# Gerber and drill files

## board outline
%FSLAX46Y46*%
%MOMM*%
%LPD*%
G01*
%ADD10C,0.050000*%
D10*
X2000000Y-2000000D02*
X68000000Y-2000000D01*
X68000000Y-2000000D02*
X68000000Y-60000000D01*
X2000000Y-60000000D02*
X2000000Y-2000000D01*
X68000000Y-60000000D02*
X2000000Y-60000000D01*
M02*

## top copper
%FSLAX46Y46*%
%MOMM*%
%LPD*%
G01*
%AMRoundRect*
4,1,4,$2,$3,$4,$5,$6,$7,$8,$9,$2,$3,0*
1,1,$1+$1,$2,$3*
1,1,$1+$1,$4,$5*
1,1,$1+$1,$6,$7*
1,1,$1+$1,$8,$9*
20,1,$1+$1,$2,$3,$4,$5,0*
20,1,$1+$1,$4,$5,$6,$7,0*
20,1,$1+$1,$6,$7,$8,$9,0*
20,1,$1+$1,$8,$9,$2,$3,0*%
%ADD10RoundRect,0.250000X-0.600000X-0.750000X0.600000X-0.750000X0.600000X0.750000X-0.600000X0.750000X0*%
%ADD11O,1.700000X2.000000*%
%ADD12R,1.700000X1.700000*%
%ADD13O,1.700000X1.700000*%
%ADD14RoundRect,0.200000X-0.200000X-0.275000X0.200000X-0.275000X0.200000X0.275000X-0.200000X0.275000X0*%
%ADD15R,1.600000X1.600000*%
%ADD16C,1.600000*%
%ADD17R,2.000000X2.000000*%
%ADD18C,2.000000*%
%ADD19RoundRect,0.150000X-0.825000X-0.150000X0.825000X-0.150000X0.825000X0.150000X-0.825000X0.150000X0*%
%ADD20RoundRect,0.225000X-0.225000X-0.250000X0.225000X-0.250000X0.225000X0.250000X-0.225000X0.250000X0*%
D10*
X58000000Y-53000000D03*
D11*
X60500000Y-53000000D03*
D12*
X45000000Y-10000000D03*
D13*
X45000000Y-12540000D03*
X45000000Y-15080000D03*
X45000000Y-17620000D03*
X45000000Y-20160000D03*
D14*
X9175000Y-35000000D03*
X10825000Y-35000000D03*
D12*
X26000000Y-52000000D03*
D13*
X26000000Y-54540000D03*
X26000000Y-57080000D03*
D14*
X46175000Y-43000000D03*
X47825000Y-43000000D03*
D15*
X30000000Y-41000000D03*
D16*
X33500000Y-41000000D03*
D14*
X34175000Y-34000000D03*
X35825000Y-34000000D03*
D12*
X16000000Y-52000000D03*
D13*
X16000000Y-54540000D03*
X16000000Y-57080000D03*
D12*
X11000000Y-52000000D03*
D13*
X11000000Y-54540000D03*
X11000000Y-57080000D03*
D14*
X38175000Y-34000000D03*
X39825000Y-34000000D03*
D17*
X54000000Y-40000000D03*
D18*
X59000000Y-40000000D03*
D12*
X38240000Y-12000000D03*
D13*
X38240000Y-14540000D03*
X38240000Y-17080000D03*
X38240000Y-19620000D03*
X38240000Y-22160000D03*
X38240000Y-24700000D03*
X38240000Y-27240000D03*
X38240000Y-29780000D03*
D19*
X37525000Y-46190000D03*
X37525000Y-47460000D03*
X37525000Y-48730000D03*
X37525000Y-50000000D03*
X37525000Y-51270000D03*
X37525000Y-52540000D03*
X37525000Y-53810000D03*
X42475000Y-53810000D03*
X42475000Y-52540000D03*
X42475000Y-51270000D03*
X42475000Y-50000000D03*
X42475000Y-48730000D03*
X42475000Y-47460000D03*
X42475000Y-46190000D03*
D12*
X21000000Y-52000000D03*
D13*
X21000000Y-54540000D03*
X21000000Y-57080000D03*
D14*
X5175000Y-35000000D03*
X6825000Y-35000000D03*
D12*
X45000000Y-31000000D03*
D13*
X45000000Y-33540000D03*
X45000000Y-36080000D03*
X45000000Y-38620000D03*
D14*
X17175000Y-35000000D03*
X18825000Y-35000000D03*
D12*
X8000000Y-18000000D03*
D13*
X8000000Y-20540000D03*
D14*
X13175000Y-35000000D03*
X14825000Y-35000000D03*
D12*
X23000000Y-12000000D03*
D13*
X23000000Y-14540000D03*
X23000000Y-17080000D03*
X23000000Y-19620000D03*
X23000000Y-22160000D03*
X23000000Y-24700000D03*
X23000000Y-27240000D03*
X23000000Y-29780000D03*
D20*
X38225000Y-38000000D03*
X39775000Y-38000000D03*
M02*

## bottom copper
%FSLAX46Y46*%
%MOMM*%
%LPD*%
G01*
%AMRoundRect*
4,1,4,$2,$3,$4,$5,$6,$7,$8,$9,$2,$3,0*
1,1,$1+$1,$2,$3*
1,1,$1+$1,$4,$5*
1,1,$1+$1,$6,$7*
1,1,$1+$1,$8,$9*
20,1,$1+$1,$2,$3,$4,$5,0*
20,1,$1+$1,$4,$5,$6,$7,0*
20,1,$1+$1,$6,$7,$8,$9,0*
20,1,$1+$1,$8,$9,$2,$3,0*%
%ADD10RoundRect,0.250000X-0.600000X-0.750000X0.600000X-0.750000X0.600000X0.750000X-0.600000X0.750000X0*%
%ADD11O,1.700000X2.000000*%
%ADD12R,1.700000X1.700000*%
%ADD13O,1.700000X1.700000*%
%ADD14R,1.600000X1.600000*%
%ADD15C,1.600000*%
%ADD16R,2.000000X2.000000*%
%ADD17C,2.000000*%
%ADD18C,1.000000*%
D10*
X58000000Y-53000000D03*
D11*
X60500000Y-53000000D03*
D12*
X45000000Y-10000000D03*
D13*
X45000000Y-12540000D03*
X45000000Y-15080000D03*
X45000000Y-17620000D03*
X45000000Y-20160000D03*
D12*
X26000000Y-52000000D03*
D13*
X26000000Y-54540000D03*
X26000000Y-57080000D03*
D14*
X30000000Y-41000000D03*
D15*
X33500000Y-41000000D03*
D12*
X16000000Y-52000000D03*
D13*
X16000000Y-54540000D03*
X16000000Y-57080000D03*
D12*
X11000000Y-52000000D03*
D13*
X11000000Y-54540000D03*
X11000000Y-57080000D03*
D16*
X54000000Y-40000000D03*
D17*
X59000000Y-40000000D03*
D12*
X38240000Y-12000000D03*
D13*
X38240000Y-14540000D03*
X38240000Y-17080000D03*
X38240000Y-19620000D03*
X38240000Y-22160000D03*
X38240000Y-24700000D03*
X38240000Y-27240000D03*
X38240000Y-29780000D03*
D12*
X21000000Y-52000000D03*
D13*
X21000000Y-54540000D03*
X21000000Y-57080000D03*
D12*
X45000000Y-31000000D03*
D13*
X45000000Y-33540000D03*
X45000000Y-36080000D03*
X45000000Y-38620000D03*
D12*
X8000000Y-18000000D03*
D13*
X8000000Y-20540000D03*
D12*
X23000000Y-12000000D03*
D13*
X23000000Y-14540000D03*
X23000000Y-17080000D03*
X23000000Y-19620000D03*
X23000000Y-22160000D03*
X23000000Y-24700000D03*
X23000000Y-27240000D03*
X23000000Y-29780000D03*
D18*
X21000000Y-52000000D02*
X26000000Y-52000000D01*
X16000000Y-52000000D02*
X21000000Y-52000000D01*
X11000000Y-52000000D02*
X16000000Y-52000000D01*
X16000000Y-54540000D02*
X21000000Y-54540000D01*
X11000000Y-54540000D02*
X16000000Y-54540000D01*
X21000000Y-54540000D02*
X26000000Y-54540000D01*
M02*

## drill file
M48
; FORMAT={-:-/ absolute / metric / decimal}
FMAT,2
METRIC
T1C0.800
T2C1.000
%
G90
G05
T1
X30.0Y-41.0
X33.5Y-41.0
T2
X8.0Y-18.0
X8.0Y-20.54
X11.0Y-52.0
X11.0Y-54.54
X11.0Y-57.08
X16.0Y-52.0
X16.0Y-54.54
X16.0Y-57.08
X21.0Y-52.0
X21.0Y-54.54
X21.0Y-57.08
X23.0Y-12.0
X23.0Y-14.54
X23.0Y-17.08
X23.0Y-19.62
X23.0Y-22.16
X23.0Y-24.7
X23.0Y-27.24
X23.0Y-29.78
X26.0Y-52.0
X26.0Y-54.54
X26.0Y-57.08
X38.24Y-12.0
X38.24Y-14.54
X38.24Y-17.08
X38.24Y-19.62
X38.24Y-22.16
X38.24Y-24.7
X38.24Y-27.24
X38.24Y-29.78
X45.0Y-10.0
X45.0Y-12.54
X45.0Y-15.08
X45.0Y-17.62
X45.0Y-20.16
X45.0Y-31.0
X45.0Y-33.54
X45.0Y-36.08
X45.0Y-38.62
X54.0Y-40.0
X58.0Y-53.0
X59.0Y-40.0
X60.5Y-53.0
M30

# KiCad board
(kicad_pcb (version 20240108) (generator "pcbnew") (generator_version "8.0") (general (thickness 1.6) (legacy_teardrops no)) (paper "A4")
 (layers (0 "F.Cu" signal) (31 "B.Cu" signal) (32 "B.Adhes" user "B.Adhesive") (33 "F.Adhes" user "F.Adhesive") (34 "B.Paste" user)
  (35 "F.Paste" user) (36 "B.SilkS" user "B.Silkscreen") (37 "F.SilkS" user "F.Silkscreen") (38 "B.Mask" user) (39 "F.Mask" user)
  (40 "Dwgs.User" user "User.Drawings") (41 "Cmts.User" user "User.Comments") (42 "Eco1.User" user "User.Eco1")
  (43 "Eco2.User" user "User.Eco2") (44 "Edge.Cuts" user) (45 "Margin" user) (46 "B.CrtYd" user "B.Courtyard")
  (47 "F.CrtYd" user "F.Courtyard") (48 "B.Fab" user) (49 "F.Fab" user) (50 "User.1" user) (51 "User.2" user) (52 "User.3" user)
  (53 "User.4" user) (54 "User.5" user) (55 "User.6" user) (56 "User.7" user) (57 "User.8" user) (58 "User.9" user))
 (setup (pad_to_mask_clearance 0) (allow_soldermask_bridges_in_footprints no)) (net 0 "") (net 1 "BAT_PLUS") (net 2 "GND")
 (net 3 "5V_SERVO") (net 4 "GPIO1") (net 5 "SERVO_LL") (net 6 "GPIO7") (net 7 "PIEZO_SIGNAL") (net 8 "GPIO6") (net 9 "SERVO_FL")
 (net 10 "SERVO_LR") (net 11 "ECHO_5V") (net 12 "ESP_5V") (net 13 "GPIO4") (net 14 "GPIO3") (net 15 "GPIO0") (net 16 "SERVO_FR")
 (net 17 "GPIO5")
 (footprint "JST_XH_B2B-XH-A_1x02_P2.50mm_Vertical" (layer "F.Cu") (at 58 53)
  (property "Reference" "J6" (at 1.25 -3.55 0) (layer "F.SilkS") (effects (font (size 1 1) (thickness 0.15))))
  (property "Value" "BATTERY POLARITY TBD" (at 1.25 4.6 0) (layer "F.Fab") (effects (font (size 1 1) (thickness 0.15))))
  (pad "1" thru_hole roundrect (at 0 0) (size 1.7 2) (drill 1) (layers "*.Cu" "*.Mask") (remove_unused_layers no)
   (roundrect_rratio 0.147059) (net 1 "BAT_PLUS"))
  (pad "2" thru_hole oval (at 2.5 0) (size 1.7 2) (drill 1) (layers "*.Cu" "*.Mask") (remove_unused_layers no) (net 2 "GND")))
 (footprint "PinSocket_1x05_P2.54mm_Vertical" (layer "F.Cu") (at 45 10)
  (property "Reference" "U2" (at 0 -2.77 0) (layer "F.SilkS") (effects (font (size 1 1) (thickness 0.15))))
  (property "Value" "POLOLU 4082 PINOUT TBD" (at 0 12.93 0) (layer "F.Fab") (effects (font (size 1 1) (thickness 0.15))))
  (pad "1" thru_hole rect (at 0 0) (size 1.7 1.7) (drill 1) (layers "*.Cu" "*.Mask") (remove_unused_layers no))
  (pad "2" thru_hole oval (at 0 2.54) (size 1.7 1.7) (drill 1) (layers "*.Cu" "*.Mask") (remove_unused_layers no) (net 1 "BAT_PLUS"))
  (pad "3" thru_hole oval (at 0 5.08) (size 1.7 1.7) (drill 1) (layers "*.Cu" "*.Mask") (remove_unused_layers no) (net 2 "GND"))
  (pad "4" thru_hole oval (at 0 7.62) (size 1.7 1.7) (drill 1) (layers "*.Cu" "*.Mask") (remove_unused_layers no) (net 2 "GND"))
  (pad "5" thru_hole oval (at 0 10.16) (size 1.7 1.7) (drill 1) (layers "*.Cu" "*.Mask") (remove_unused_layers no) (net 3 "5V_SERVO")))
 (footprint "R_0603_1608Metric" (layer "F.Cu") (at 10 35)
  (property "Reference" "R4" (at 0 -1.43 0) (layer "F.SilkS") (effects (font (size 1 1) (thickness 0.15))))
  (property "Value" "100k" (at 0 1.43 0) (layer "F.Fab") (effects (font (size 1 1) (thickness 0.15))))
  (pad "1" smd roundrect (at -0.825 0) (size 0.8 0.95) (layers "F.Cu" "F.Paste" "F.Mask") (roundrect_rratio 0.25) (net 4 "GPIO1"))
  (pad "2" smd roundrect (at 0.825 0) (size 0.8 0.95) (layers "F.Cu" "F.Paste" "F.Mask") (roundrect_rratio 0.25) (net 2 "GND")))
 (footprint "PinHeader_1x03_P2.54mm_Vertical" (layer "F.Cu") (at 26 52)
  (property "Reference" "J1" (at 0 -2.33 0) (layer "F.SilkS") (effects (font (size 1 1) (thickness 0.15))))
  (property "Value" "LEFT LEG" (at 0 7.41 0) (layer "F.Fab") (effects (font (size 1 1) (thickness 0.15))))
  (pad "1" thru_hole rect (at 0 0) (size 1.7 1.7) (drill 1) (layers "*.Cu" "*.Mask") (remove_unused_layers no) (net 2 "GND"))
  (pad "2" thru_hole oval (at 0 2.54) (size 1.7 1.7) (drill 1) (layers "*.Cu" "*.Mask") (remove_unused_layers no) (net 3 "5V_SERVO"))
  (pad "3" thru_hole oval (at 0 5.08) (size 1.7 1.7) (drill 1) (layers "*.Cu" "*.Mask") (remove_unused_layers no) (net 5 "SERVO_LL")))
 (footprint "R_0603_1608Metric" (layer "F.Cu") (at 47 43)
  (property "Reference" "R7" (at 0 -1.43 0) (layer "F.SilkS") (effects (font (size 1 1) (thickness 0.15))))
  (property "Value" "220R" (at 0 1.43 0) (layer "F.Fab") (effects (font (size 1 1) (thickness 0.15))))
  (pad "1" smd roundrect (at -0.825 0) (size 0.8 0.95) (layers "F.Cu" "F.Paste" "F.Mask") (roundrect_rratio 0.25) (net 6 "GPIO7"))
  (pad "2" smd roundrect (at 0.825 0) (size 0.8 0.95) (layers "F.Cu" "F.Paste" "F.Mask") (roundrect_rratio 0.25) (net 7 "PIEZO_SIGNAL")))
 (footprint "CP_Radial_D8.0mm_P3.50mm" (layer "F.Cu") (at 30 41)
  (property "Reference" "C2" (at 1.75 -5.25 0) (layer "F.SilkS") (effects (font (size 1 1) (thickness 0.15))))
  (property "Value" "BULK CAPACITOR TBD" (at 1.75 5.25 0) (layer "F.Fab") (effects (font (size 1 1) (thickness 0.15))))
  (pad "1" thru_hole rect (at 0 0) (size 1.6 1.6) (drill 0.8) (layers "*.Cu" "*.Mask") (remove_unused_layers no) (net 3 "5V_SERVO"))
  (pad "2" thru_hole circle (at 3.5 0) (size 1.6 1.6) (drill 0.8) (layers "*.Cu" "*.Mask") (remove_unused_layers no) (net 2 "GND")))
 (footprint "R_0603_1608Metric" (layer "F.Cu") (at 35 34)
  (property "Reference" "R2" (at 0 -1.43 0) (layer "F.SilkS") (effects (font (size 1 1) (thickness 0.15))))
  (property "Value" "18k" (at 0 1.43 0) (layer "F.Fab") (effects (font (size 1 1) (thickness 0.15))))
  (pad "1" smd roundrect (at -0.825 0) (size 0.8 0.95) (layers "F.Cu" "F.Paste" "F.Mask") (roundrect_rratio 0.25) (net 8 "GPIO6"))
  (pad "2" smd roundrect (at 0.825 0) (size 0.8 0.95) (layers "F.Cu" "F.Paste" "F.Mask") (roundrect_rratio 0.25) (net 2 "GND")))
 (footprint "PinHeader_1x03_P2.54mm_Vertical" (layer "F.Cu") (at 16 52)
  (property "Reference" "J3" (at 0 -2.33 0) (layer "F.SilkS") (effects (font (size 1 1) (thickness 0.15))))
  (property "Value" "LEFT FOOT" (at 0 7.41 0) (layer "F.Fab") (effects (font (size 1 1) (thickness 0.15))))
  (pad "1" thru_hole rect (at 0 0) (size 1.7 1.7) (drill 1) (layers "*.Cu" "*.Mask") (remove_unused_layers no) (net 2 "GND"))
  (pad "2" thru_hole oval (at 0 2.54) (size 1.7 1.7) (drill 1) (layers "*.Cu" "*.Mask") (remove_unused_layers no) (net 3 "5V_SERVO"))
  (pad "3" thru_hole oval (at 0 5.08) (size 1.7 1.7) (drill 1) (layers "*.Cu" "*.Mask") (remove_unused_layers no) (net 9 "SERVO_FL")))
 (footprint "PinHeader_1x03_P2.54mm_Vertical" (layer "F.Cu") (at 11 52)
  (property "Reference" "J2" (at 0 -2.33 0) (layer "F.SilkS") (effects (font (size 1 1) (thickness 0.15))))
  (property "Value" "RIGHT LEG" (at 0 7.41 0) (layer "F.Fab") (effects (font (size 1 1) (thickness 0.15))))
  (pad "1" thru_hole rect (at 0 0) (size 1.7 1.7) (drill 1) (layers "*.Cu" "*.Mask") (remove_unused_layers no) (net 2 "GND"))
  (pad "2" thru_hole oval (at 0 2.54) (size 1.7 1.7) (drill 1) (layers "*.Cu" "*.Mask") (remove_unused_layers no) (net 3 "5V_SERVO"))
  (pad "3" thru_hole oval (at 0 5.08) (size 1.7 1.7) (drill 1) (layers "*.Cu" "*.Mask") (remove_unused_layers no) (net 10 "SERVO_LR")))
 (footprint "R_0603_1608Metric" (layer "F.Cu") (at 39 34)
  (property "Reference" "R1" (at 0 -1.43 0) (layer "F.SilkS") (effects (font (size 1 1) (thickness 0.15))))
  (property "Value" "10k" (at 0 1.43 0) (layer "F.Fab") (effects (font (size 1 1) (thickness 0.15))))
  (pad "1" smd roundrect (at -0.825 0) (size 0.8 0.95) (layers "F.Cu" "F.Paste" "F.Mask") (roundrect_rratio 0.25) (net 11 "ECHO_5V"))
  (pad "2" smd roundrect (at 0.825 0) (size 0.8 0.95) (layers "F.Cu" "F.Paste" "F.Mask") (roundrect_rratio 0.25) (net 8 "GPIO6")))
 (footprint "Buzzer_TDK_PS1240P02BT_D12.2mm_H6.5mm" (layer "F.Cu") (at 54 40)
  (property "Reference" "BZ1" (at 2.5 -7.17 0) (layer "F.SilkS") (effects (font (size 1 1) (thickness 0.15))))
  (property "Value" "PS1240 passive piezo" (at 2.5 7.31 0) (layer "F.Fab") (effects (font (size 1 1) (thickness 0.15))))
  (pad "1" thru_hole rect (at 0 0) (size 2 2) (drill 1) (layers "*.Cu" "*.Mask") (remove_unused_layers no) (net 7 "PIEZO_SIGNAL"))
  (pad "2" thru_hole circle (at 5 0) (size 2 2) (drill 1) (layers "*.Cu" "*.Mask") (remove_unused_layers no) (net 2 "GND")))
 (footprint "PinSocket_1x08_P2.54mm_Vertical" (layer "F.Cu") (at 38.24 12)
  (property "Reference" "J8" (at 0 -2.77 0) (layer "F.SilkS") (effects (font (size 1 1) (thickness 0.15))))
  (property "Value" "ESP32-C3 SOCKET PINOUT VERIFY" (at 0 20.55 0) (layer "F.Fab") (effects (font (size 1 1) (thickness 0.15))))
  (pad "1" thru_hole rect (at 0 0) (size 1.7 1.7) (drill 1) (layers "*.Cu" "*.Mask") (remove_unused_layers no) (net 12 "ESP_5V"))
  (pad "2" thru_hole oval (at 0 2.54) (size 1.7 1.7) (drill 1) (layers "*.Cu" "*.Mask") (remove_unused_layers no) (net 2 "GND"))
  (pad "3" thru_hole oval (at 0 5.08) (size 1.7 1.7) (drill 1) (layers "*.Cu" "*.Mask") (remove_unused_layers no))
  (pad "4" thru_hole oval (at 0 7.62) (size 1.7 1.7) (drill 1) (layers "*.Cu" "*.Mask") (remove_unused_layers no) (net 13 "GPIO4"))
  (pad "5" thru_hole oval (at 0 10.16) (size 1.7 1.7) (drill 1) (layers "*.Cu" "*.Mask") (remove_unused_layers no) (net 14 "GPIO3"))
  (pad "6" thru_hole oval (at 0 12.7) (size 1.7 1.7) (drill 1) (layers "*.Cu" "*.Mask") (remove_unused_layers no))
  (pad "7" thru_hole oval (at 0 15.24) (size 1.7 1.7) (drill 1) (layers "*.Cu" "*.Mask") (remove_unused_layers no) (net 4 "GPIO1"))
  (pad "8" thru_hole oval (at 0 17.78) (size 1.7 1.7) (drill 1) (layers "*.Cu" "*.Mask") (remove_unused_layers no) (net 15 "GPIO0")))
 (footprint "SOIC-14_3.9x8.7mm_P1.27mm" (layer "F.Cu") (at 40 50)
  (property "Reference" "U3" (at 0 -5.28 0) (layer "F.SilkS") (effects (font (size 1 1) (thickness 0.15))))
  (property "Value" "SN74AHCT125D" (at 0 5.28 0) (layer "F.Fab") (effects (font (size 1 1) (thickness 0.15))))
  (pad "1" smd roundrect (at -2.475 -3.81) (size 1.95 0.6) (layers "F.Cu" "F.Paste" "F.Mask") (roundrect_rratio 0.25) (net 2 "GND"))
  (pad "2" smd roundrect (at -2.475 -2.54) (size 1.95 0.6) (layers "F.Cu" "F.Paste" "F.Mask") (roundrect_rratio 0.25) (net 15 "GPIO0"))
  (pad "3" smd roundrect (at -2.475 -1.27) (size 1.95 0.6) (layers "F.Cu" "F.Paste" "F.Mask") (roundrect_rratio 0.25) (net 5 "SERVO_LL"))
  (pad "4" smd roundrect (at -2.475 0) (size 1.95 0.6) (layers "F.Cu" "F.Paste" "F.Mask") (roundrect_rratio 0.25) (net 2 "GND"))
  (pad "5" smd roundrect (at -2.475 1.27) (size 1.95 0.6) (layers "F.Cu" "F.Paste" "F.Mask") (roundrect_rratio 0.25) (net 4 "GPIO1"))
  (pad "6" smd roundrect (at -2.475 2.54) (size 1.95 0.6) (layers "F.Cu" "F.Paste" "F.Mask") (roundrect_rratio 0.25) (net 10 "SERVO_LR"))
  (pad "7" smd roundrect (at -2.475 3.81) (size 1.95 0.6) (layers "F.Cu" "F.Paste" "F.Mask") (roundrect_rratio 0.25) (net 2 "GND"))
  (pad "8" smd roundrect (at 2.475 3.81) (size 1.95 0.6) (layers "F.Cu" "F.Paste" "F.Mask") (roundrect_rratio 0.25) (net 9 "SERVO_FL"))
  (pad "9" smd roundrect (at 2.475 2.54) (size 1.95 0.6) (layers "F.Cu" "F.Paste" "F.Mask") (roundrect_rratio 0.25) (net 14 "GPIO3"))
  (pad "10" smd roundrect (at 2.475 1.27) (size 1.95 0.6) (layers "F.Cu" "F.Paste" "F.Mask") (roundrect_rratio 0.25) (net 2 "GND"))
  (pad "11" smd roundrect (at 2.475 0) (size 1.95 0.6) (layers "F.Cu" "F.Paste" "F.Mask") (roundrect_rratio 0.25) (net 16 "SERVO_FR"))
  (pad "12" smd roundrect (at 2.475 -1.27) (size 1.95 0.6) (layers "F.Cu" "F.Paste" "F.Mask") (roundrect_rratio 0.25) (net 13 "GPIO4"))
  (pad "13" smd roundrect (at 2.475 -2.54) (size 1.95 0.6) (layers "F.Cu" "F.Paste" "F.Mask") (roundrect_rratio 0.25) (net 2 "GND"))
  (pad "14" smd roundrect (at 2.475 -3.81) (size 1.95 0.6) (layers "F.Cu" "F.Paste" "F.Mask") (roundrect_rratio 0.25) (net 3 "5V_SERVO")))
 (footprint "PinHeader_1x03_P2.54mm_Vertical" (layer "F.Cu") (at 21 52)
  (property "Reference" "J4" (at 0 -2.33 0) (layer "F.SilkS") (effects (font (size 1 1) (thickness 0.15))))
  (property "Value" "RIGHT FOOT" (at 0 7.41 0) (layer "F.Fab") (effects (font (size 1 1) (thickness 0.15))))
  (pad "1" thru_hole rect (at 0 0) (size 1.7 1.7) (drill 1) (layers "*.Cu" "*.Mask") (remove_unused_layers no) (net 2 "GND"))
  (pad "2" thru_hole oval (at 0 2.54) (size 1.7 1.7) (drill 1) (layers "*.Cu" "*.Mask") (remove_unused_layers no) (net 3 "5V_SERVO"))
  (pad "3" thru_hole oval (at 0 5.08) (size 1.7 1.7) (drill 1) (layers "*.Cu" "*.Mask") (remove_unused_layers no) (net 16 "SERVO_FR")))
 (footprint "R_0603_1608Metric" (layer "F.Cu") (at 6 35)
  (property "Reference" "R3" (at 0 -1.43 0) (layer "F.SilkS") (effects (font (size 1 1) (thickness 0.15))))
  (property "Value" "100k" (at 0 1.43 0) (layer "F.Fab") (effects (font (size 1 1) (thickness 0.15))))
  (pad "1" smd roundrect (at -0.825 0) (size 0.8 0.95) (layers "F.Cu" "F.Paste" "F.Mask") (roundrect_rratio 0.25) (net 15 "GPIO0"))
  (pad "2" smd roundrect (at 0.825 0) (size 0.8 0.95) (layers "F.Cu" "F.Paste" "F.Mask") (roundrect_rratio 0.25) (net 2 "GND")))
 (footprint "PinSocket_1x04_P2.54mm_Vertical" (layer "F.Cu") (at 45 31)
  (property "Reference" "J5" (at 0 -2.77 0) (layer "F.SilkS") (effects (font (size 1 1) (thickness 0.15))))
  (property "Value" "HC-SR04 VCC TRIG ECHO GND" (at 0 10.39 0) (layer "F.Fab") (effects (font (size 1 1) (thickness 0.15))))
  (pad "1" thru_hole rect (at 0 0) (size 1.7 1.7) (drill 1) (layers "*.Cu" "*.Mask") (remove_unused_layers no) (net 3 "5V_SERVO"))
  (pad "2" thru_hole oval (at 0 2.54) (size 1.7 1.7) (drill 1) (layers "*.Cu" "*.Mask") (remove_unused_layers no) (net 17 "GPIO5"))
  (pad "3" thru_hole oval (at 0 5.08) (size 1.7 1.7) (drill 1) (layers "*.Cu" "*.Mask") (remove_unused_layers no) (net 11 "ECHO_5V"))
  (pad "4" thru_hole oval (at 0 7.62) (size 1.7 1.7) (drill 1) (layers "*.Cu" "*.Mask") (remove_unused_layers no) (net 2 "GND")))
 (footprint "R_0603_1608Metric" (layer "F.Cu") (at 18 35)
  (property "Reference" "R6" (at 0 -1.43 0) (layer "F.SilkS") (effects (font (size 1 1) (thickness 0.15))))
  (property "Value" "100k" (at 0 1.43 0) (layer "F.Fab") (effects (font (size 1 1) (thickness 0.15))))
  (pad "1" smd roundrect (at -0.825 0) (size 0.8 0.95) (layers "F.Cu" "F.Paste" "F.Mask") (roundrect_rratio 0.25) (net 13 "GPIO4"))
  (pad "2" smd roundrect (at 0.825 0) (size 0.8 0.95) (layers "F.Cu" "F.Paste" "F.Mask") (roundrect_rratio 0.25) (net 2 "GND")))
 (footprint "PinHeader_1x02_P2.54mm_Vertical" (layer "F.Cu") (at 8 18)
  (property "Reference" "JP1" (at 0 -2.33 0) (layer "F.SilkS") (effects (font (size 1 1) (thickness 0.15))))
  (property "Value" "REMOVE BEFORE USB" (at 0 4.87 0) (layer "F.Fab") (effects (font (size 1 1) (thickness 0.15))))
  (pad "1" thru_hole rect (at 0 0) (size 1.7 1.7) (drill 1) (layers "*.Cu" "*.Mask") (remove_unused_layers no) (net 3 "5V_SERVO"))
  (pad "2" thru_hole oval (at 0 2.54) (size 1.7 1.7) (drill 1) (layers "*.Cu" "*.Mask") (remove_unused_layers no) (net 12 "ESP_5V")))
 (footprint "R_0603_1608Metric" (layer "F.Cu") (at 14 35)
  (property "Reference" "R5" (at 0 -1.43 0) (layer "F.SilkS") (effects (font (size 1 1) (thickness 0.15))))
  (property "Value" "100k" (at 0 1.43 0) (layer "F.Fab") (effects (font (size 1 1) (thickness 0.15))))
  (pad "1" smd roundrect (at -0.825 0) (size 0.8 0.95) (layers "F.Cu" "F.Paste" "F.Mask") (roundrect_rratio 0.25) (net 14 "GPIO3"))
  (pad "2" smd roundrect (at 0.825 0) (size 0.8 0.95) (layers "F.Cu" "F.Paste" "F.Mask") (roundrect_rratio 0.25) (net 2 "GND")))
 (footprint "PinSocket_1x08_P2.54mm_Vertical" (layer "F.Cu") (at 23 12)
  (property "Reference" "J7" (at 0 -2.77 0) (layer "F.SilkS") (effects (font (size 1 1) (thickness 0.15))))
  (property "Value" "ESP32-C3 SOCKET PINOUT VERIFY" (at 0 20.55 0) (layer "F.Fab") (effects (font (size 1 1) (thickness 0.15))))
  (pad "1" thru_hole rect (at 0 0) (size 1.7 1.7) (drill 1) (layers "*.Cu" "*.Mask") (remove_unused_layers no) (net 17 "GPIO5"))
  (pad "2" thru_hole oval (at 0 2.54) (size 1.7 1.7) (drill 1) (layers "*.Cu" "*.Mask") (remove_unused_layers no) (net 8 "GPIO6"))
  (pad "3" thru_hole oval (at 0 5.08) (size 1.7 1.7) (drill 1) (layers "*.Cu" "*.Mask") (remove_unused_layers no) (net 6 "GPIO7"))
  (pad "4" thru_hole oval (at 0 7.62) (size 1.7 1.7) (drill 1) (layers "*.Cu" "*.Mask") (remove_unused_layers no))
  (pad "5" thru_hole oval (at 0 10.16) (size 1.7 1.7) (drill 1) (layers "*.Cu" "*.Mask") (remove_unused_layers no))
  (pad "6" thru_hole oval (at 0 12.7) (size 1.7 1.7) (drill 1) (layers "*.Cu" "*.Mask") (remove_unused_layers no))
  (pad "7" thru_hole oval (at 0 15.24) (size 1.7 1.7) (drill 1) (layers "*.Cu" "*.Mask") (remove_unused_layers no))
  (pad "8" thru_hole oval (at 0 17.78) (size 1.7 1.7) (drill 1) (layers "*.Cu" "*.Mask") (remove_unused_layers no)))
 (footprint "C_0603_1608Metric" (layer "F.Cu") (at 39 38)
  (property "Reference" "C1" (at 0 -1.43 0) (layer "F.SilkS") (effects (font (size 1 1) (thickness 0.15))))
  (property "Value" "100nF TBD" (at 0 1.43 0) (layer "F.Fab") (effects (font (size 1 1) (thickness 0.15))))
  (pad "1" smd roundrect (at -0.775 0) (size 0.9 0.95) (layers "F.Cu" "F.Paste" "F.Mask") (roundrect_rratio 0.25) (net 3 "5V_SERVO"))
  (pad "2" smd roundrect (at 0.775 0) (size 0.9 0.95) (layers "F.Cu" "F.Paste" "F.Mask") (roundrect_rratio 0.25) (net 2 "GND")))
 (gr_line (start 2 2) (end 68 2) (stroke (width 0.05) (type default)) (layer "Edge.Cuts"))
 (gr_line (start 68 2) (end 68 60) (stroke (width 0.05) (type default)) (layer "Edge.Cuts"))
 (gr_line (start 2 60) (end 2 2) (stroke (width 0.05) (type default)) (layer "Edge.Cuts"))
 (gr_line (start 68 60) (end 2 60) (stroke (width 0.05) (type default)) (layer "Edge.Cuts"))
 (segment (start 21 52) (end 26 52) (width 1) (layer "B.Cu") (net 2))
 (segment (start 16 52) (end 21 52) (width 1) (layer "B.Cu") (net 2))
 (segment (start 11 52) (end 16 52) (width 1) (layer "B.Cu") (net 2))
 (segment (start 16 54.54) (end 21 54.54) (width 1) (layer "B.Cu") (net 3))
 (segment (start 11 54.54) (end 16 54.54) (width 1) (layer "B.Cu") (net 3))
 (segment (start 21 54.54) (end 26 54.54) (width 1) (layer "B.Cu") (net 3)))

